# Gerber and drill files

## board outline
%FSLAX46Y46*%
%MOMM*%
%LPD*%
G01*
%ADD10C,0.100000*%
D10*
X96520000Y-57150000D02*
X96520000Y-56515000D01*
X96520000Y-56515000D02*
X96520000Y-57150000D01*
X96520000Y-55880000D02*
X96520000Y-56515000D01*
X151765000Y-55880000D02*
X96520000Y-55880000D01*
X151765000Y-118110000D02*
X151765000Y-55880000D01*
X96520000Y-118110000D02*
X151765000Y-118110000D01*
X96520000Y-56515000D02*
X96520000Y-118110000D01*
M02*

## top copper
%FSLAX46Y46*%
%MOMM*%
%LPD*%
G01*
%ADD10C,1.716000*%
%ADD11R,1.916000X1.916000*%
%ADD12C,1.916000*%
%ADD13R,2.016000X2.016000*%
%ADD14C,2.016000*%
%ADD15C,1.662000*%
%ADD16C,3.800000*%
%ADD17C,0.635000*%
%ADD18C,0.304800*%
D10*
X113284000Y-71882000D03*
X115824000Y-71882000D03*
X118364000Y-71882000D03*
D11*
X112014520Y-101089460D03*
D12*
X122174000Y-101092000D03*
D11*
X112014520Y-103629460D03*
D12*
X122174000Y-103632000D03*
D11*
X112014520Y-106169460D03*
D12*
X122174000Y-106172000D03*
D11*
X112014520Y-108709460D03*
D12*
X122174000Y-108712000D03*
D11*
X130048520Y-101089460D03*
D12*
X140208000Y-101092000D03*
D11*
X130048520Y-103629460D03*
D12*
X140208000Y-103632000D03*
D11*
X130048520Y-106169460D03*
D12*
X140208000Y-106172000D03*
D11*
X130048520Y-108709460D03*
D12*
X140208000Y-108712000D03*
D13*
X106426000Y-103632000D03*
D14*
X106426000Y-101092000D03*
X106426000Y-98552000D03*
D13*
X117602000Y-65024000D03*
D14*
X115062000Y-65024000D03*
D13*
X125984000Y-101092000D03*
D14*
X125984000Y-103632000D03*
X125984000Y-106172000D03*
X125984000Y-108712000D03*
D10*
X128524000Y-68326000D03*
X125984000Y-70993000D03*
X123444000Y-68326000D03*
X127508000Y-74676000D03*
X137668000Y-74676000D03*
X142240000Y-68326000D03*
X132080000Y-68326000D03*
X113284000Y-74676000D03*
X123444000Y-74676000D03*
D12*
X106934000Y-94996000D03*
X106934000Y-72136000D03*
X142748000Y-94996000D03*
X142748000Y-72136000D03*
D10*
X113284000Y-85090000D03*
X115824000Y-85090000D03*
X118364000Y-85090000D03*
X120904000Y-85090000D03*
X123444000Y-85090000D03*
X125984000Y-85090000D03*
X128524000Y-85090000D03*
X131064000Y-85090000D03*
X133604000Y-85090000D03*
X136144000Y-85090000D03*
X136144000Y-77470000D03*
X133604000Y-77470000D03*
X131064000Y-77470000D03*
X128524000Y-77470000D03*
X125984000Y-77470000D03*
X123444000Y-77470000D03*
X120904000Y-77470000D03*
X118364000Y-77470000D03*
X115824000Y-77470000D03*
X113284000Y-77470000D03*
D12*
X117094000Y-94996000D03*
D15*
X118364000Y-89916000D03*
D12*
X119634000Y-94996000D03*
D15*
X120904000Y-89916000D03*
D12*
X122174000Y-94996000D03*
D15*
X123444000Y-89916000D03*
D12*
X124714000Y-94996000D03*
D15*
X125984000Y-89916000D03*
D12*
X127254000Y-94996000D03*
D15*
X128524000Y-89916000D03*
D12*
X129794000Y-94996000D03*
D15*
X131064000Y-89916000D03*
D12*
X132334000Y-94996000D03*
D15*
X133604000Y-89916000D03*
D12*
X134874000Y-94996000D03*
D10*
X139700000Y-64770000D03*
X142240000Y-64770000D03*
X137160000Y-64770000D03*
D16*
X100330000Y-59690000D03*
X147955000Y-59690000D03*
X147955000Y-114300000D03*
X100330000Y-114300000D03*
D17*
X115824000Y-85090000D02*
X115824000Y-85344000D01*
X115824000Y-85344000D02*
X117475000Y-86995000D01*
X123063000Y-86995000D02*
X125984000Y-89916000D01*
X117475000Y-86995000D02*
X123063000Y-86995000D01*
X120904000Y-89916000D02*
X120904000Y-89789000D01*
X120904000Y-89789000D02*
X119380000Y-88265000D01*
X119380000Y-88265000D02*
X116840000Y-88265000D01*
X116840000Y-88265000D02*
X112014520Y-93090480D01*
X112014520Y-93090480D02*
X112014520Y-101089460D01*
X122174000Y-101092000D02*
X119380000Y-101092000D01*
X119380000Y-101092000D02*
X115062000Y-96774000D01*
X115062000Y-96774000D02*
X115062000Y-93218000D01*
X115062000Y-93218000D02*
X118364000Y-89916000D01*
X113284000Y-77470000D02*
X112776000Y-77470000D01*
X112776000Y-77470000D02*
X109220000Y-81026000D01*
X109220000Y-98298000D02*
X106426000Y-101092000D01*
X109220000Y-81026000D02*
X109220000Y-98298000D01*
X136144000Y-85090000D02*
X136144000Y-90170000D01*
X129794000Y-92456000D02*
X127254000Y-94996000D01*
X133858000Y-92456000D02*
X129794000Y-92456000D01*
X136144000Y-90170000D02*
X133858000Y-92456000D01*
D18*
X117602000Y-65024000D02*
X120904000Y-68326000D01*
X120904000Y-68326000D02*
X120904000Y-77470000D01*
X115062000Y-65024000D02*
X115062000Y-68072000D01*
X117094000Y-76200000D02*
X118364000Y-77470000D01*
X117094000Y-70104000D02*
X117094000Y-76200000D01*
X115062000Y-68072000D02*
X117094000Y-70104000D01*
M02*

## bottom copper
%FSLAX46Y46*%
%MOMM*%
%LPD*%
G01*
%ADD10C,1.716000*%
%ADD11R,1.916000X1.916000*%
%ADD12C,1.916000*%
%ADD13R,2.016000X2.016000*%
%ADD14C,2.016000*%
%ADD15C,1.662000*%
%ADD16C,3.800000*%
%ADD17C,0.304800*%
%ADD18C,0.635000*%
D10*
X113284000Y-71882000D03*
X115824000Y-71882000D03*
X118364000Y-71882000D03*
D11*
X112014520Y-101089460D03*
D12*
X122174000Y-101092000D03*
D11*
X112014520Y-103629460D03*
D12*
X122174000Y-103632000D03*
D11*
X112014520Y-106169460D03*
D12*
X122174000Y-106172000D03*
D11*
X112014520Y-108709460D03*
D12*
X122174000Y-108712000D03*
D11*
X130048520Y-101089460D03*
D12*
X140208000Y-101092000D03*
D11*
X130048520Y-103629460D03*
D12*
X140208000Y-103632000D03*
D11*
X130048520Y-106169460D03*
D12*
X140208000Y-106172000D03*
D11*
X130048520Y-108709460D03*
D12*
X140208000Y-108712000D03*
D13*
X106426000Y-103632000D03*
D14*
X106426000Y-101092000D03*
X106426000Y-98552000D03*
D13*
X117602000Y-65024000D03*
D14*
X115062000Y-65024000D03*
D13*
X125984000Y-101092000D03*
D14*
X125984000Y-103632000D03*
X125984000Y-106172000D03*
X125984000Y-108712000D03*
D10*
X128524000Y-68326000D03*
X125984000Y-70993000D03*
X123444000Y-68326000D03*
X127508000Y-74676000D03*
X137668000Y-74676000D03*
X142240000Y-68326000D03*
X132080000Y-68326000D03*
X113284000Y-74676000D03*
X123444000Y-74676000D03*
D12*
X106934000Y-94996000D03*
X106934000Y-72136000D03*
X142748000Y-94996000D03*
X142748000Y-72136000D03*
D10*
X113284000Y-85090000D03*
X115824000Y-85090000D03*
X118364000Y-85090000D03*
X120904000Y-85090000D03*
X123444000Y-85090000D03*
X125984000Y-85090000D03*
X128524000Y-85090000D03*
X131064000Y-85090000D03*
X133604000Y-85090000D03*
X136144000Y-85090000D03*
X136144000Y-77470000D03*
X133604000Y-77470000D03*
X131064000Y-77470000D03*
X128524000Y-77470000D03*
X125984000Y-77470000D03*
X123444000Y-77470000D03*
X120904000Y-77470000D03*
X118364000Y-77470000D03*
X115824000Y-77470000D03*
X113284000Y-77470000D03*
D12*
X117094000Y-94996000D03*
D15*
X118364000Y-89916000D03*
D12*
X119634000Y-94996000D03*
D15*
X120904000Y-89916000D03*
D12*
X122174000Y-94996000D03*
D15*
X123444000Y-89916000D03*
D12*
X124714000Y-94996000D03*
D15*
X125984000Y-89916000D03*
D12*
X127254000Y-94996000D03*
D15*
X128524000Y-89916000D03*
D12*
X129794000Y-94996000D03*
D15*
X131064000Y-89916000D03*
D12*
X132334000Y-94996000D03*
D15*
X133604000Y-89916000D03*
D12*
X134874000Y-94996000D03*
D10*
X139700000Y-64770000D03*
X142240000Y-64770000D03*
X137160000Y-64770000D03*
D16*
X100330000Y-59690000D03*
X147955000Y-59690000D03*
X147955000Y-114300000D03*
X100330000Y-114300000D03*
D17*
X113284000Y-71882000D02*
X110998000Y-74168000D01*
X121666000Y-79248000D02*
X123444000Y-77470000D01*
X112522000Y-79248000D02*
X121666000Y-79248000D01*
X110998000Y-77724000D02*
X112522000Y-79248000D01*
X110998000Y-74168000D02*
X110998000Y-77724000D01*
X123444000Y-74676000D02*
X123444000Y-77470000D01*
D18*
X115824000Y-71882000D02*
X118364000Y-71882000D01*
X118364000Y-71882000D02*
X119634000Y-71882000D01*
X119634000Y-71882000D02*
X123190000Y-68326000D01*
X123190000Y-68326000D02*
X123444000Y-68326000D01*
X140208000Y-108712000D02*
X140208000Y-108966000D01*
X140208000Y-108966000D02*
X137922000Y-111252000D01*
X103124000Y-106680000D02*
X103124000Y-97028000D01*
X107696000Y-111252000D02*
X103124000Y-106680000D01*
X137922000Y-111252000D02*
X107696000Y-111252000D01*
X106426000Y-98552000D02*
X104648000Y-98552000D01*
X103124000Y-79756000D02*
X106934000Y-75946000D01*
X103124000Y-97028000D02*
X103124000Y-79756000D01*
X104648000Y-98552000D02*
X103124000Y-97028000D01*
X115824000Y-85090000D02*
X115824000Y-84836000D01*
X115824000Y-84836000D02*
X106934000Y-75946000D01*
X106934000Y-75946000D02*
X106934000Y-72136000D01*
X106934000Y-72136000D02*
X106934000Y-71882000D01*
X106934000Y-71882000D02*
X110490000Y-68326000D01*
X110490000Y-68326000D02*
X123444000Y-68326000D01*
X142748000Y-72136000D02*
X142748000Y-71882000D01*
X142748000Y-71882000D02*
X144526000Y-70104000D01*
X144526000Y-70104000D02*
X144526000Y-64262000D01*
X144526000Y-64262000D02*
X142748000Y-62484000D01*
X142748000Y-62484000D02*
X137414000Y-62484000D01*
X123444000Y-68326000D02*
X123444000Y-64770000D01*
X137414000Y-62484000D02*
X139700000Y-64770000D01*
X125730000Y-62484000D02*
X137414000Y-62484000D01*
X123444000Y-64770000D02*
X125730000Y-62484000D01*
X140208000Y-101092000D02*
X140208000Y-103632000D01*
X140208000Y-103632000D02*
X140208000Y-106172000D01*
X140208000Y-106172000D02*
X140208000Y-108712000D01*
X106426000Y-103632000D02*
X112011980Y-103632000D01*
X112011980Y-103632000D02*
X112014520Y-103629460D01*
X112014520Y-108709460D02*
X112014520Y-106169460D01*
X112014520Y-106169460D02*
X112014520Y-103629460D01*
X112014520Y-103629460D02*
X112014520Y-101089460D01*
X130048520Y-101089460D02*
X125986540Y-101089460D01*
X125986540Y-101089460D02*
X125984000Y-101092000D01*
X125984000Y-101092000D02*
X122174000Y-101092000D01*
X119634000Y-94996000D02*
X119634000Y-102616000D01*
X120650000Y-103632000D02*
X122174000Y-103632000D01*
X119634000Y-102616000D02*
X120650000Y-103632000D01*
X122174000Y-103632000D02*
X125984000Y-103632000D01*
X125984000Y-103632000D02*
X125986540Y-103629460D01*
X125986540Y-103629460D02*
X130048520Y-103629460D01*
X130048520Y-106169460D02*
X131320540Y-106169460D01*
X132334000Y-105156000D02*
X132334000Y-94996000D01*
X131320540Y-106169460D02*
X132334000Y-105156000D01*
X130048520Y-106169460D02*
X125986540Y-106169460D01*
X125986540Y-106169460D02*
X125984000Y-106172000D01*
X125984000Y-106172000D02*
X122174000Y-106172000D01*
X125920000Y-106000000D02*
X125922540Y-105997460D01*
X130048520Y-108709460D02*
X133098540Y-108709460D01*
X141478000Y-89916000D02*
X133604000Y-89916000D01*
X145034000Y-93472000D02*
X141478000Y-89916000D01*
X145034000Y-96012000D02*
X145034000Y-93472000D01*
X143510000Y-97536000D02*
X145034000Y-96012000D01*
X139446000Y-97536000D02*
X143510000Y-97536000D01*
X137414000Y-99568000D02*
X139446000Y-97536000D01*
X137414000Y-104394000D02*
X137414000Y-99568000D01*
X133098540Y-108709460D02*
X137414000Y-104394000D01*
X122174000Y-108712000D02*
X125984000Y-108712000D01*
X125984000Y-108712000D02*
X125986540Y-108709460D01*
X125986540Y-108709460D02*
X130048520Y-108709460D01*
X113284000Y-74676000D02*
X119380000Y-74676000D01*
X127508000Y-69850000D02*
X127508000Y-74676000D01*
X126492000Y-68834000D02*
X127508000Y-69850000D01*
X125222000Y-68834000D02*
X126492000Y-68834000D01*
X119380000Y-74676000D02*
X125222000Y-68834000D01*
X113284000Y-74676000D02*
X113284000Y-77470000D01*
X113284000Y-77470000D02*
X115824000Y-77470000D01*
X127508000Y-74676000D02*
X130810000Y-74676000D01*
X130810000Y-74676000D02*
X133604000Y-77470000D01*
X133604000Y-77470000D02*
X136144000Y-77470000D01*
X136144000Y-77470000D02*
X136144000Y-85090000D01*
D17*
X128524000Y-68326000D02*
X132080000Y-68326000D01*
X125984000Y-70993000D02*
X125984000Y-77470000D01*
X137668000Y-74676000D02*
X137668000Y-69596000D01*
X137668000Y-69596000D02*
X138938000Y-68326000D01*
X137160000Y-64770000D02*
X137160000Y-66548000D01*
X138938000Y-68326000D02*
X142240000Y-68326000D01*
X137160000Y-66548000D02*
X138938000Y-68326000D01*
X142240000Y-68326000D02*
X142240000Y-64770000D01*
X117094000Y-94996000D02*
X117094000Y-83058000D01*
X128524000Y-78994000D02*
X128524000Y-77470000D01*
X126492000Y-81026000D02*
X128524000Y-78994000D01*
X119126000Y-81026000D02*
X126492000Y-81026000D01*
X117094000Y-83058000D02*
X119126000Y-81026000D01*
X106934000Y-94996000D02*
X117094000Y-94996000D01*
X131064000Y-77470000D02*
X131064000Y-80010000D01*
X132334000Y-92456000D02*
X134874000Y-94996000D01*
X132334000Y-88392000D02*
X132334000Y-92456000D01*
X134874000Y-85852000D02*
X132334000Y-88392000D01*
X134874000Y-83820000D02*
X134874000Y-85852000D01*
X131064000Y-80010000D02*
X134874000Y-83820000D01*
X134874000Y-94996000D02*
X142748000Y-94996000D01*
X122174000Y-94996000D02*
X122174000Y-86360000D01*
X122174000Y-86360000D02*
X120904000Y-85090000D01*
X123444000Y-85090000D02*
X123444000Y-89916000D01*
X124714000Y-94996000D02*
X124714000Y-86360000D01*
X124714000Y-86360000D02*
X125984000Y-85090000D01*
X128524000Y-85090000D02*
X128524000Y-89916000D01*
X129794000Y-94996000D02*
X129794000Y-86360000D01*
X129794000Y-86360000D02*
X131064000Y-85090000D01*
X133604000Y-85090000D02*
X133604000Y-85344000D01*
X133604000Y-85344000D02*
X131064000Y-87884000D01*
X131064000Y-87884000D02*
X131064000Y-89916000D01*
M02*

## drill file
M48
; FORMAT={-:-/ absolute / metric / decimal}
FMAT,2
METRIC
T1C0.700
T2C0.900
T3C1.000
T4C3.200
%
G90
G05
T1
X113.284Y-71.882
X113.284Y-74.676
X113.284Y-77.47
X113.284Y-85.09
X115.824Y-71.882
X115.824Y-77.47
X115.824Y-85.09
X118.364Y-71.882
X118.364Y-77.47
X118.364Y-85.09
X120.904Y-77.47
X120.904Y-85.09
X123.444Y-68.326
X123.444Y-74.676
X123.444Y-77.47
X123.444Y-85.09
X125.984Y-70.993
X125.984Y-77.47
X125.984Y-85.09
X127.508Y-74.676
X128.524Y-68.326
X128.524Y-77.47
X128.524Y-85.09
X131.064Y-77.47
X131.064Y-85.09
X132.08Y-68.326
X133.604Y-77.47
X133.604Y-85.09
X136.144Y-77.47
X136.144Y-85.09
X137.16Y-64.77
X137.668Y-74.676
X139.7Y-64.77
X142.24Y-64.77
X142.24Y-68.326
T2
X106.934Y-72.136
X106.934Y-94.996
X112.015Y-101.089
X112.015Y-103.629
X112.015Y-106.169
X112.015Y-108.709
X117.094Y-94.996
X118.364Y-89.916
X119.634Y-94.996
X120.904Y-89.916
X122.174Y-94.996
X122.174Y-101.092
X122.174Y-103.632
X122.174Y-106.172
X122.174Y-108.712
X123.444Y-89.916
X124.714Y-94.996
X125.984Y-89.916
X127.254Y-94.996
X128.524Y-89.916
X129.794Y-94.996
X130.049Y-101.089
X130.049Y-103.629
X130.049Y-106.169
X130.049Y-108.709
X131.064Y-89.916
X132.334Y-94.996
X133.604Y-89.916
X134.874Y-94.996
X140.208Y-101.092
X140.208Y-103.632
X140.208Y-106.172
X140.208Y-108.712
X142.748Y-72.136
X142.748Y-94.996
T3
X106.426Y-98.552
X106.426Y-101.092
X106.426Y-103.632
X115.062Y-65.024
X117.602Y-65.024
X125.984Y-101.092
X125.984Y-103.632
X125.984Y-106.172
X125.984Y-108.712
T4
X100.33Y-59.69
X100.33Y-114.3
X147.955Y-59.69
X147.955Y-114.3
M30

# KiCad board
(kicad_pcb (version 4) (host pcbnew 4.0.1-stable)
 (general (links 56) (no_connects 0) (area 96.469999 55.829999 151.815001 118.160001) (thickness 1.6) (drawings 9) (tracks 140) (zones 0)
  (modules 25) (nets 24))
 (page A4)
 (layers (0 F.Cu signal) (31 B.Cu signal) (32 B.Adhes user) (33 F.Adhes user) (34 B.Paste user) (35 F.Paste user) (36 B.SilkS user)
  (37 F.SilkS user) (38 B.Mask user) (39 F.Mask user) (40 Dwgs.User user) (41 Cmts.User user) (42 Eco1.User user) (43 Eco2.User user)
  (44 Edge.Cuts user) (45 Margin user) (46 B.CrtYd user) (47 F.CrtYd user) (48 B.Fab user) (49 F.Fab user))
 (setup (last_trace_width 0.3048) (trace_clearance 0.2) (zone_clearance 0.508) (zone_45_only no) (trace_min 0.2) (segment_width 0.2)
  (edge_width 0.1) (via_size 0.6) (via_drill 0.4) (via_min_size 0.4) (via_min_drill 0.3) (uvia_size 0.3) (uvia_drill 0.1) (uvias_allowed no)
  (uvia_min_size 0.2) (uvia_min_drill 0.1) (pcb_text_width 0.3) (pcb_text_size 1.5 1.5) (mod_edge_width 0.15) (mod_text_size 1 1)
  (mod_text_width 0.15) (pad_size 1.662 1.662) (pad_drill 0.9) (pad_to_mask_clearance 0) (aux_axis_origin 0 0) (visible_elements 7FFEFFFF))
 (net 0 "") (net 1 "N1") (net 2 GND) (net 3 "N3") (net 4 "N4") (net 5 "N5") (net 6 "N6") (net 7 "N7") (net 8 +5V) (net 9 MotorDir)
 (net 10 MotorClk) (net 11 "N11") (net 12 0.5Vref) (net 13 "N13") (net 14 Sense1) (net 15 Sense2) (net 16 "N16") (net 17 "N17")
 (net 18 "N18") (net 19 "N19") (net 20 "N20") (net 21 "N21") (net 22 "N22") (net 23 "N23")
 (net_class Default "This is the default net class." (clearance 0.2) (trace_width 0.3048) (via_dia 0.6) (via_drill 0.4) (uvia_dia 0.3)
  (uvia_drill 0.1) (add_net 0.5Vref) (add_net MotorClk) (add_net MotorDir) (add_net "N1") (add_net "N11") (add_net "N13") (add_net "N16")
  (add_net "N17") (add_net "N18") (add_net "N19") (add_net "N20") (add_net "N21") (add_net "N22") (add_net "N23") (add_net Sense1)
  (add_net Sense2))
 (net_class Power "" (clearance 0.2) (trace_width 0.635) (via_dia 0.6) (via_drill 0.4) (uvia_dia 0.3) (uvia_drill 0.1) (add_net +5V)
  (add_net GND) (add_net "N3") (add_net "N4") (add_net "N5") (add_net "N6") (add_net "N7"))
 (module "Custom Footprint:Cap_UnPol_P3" (layer F.Cu) (at 113.284 71.882 90)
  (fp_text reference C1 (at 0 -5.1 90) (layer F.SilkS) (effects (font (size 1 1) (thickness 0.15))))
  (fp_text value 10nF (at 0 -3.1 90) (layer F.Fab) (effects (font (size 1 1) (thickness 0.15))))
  (pad 1 thru_hole circle (at 0 0 90) (size 1.716 1.716) (drill 0.7) (layers *.Cu *.Mask F.SilkS) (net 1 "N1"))
  (pad 2 thru_hole circle (at 0 2.54 90) (size 1.716 1.716) (drill 0.7) (layers *.Cu *.Mask F.SilkS) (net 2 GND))
  (pad 2 thru_hole circle (at 0 5.08 90) (size 1.716 1.716) (drill 0.7) (layers *.Cu *.Mask F.SilkS) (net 2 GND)))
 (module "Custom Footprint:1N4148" (layer F.Cu) (at 112.014 101.092)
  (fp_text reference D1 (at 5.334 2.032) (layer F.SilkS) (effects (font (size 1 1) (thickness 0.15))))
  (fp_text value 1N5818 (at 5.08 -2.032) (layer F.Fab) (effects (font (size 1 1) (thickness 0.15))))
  (pad 1 thru_hole rect (at 0.00052 -0.00254 180) (size 1.916 1.916) (drill 0.9) (layers *.Cu *.Mask F.SilkS) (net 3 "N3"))
  (pad 2 thru_hole circle (at 10.16 0) (size 1.916 1.916) (drill 0.9) (layers *.Cu *.Mask F.SilkS) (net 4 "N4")))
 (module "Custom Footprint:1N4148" (layer F.Cu) (at 112.014 103.632)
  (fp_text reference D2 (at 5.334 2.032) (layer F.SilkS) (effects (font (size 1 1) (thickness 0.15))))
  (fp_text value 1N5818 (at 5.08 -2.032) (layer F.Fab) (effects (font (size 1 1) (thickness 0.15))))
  (pad 1 thru_hole rect (at 0.00052 -0.00254 180) (size 1.916 1.916) (drill 0.9) (layers *.Cu *.Mask F.SilkS) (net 3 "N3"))
  (pad 2 thru_hole circle (at 10.16 0) (size 1.916 1.916) (drill 0.9) (layers *.Cu *.Mask F.SilkS) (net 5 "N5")))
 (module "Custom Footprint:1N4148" (layer F.Cu) (at 112.014 106.172)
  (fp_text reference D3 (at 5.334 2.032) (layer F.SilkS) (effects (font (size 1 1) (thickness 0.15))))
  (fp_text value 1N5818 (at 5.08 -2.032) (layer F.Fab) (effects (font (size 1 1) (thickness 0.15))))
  (pad 1 thru_hole rect (at 0.00052 -0.00254 180) (size 1.916 1.916) (drill 0.9) (layers *.Cu *.Mask F.SilkS) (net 3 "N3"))
  (pad 2 thru_hole circle (at 10.16 0) (size 1.916 1.916) (drill 0.9) (layers *.Cu *.Mask F.SilkS) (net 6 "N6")))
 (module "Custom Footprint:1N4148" (layer F.Cu) (at 112.014 108.712)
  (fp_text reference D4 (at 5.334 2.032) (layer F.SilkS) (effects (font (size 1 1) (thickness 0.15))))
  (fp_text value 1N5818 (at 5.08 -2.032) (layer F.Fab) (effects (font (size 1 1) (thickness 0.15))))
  (pad 1 thru_hole rect (at 0.00052 -0.00254 180) (size 1.916 1.916) (drill 0.9) (layers *.Cu *.Mask F.SilkS) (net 3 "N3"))
  (pad 2 thru_hole circle (at 10.16 0) (size 1.916 1.916) (drill 0.9) (layers *.Cu *.Mask F.SilkS) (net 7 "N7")))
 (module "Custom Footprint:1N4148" (layer F.Cu) (at 130.048 101.092)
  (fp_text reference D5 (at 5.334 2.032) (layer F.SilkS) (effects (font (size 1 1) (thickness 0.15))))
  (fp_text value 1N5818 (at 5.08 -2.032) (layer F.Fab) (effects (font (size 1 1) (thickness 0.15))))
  (pad 1 thru_hole rect (at 0.00052 -0.00254 180) (size 1.916 1.916) (drill 0.9) (layers *.Cu *.Mask F.SilkS) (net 4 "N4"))
  (pad 2 thru_hole circle (at 10.16 0) (size 1.916 1.916) (drill 0.9) (layers *.Cu *.Mask F.SilkS) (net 2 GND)))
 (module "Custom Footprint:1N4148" (layer F.Cu) (at 130.048 103.632)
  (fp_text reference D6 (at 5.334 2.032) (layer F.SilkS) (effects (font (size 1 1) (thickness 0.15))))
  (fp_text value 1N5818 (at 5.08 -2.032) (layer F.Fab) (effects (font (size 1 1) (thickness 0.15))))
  (pad 1 thru_hole rect (at 0.00052 -0.00254 180) (size 1.916 1.916) (drill 0.9) (layers *.Cu *.Mask F.SilkS) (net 5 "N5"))
  (pad 2 thru_hole circle (at 10.16 0) (size 1.916 1.916) (drill 0.9) (layers *.Cu *.Mask F.SilkS) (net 2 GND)))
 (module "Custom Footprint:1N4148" (layer F.Cu) (at 130.048 106.172)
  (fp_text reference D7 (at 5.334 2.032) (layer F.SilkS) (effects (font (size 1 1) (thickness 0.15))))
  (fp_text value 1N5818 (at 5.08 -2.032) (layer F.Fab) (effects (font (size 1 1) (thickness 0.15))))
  (pad 1 thru_hole rect (at 0.00052 -0.00254 180) (size 1.916 1.916) (drill 0.9) (layers *.Cu *.Mask F.SilkS) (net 6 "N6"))
  (pad 2 thru_hole circle (at 10.16 0) (size 1.916 1.916) (drill 0.9) (layers *.Cu *.Mask F.SilkS) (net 2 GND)))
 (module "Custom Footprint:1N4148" (layer F.Cu) (at 130.048 108.712)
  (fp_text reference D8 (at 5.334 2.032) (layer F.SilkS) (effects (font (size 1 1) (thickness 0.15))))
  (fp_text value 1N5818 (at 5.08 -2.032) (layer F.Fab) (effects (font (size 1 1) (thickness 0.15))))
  (pad 1 thru_hole rect (at 0.00052 -0.00254 180) (size 1.916 1.916) (drill 0.9) (layers *.Cu *.Mask F.SilkS) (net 7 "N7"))
  (pad 2 thru_hole circle (at 10.16 0) (size 1.916 1.916) (drill 0.9) (layers *.Cu *.Mask F.SilkS) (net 2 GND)))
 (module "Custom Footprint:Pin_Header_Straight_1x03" (layer F.Cu) (at 106.426 103.632 180)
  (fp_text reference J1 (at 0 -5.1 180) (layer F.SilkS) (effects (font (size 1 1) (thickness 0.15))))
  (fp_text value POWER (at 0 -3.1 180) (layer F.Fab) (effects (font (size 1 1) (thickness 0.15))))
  (pad 1 thru_hole rect (at 0 0 180) (size 2.016 2.016) (drill 1) (layers *.Cu *.Mask F.SilkS) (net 3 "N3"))
  (pad 2 thru_hole circle (at 0 2.54 180) (size 2.016 2.016) (drill 1) (layers *.Cu *.Mask F.SilkS) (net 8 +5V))
  (pad 3 thru_hole circle (at 0 5.08 180) (size 2.016 2.016) (drill 1) (layers *.Cu *.Mask F.SilkS) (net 2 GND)))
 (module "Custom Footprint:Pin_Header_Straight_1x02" (layer F.Cu) (at 117.602 65.024 270)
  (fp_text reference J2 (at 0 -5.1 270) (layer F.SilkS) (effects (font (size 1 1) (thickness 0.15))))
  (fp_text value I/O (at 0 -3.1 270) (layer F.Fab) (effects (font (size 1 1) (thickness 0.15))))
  (pad 1 thru_hole rect (at 0 0 270) (size 2.016 2.016) (drill 1) (layers *.Cu *.Mask F.SilkS) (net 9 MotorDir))
  (pad 2 thru_hole circle (at 0 2.54 270) (size 2.016 2.016) (drill 1) (layers *.Cu *.Mask F.SilkS) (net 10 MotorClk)))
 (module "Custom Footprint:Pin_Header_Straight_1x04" (layer F.Cu) (at 125.984 101.092)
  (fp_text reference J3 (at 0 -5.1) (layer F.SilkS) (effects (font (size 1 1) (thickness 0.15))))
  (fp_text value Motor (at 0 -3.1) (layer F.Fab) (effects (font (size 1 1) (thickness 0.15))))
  (pad 1 thru_hole rect (at 0 0) (size 2.016 2.016) (drill 1) (layers *.Cu *.Mask F.SilkS) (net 4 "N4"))
  (pad 2 thru_hole circle (at 0 2.54) (size 2.016 2.016) (drill 1) (layers *.Cu *.Mask F.SilkS) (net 5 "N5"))
  (pad 3 thru_hole circle (at 0 5.08) (size 2.016 2.016) (drill 1) (layers *.Cu *.Mask F.SilkS) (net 6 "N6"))
  (pad 4 thru_hole circle (at 0 7.62) (size 2.016 2.016) (drill 1) (layers *.Cu *.Mask F.SilkS) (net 7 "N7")))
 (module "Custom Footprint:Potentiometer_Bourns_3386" (layer F.Cu) (at 128.524 68.326)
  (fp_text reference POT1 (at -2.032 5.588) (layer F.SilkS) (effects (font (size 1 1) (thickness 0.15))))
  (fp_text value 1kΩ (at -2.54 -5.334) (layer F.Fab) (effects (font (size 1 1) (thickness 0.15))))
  (pad 1 thru_hole circle (at 0 0) (size 1.716 1.716) (drill 0.7) (layers *.Cu *.Mask F.SilkS) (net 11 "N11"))
  (pad 2 thru_hole circle (at -2.54 2.667) (size 1.716 1.716) (drill 0.7) (layers *.Cu *.Mask F.SilkS) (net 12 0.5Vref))
  (pad 3 thru_hole circle (at -5.08 0) (size 1.716 1.716) (drill 0.7) (layers *.Cu *.Mask F.SilkS) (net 2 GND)))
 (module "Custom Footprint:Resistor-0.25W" (layer F.Cu) (at 127.508 74.676)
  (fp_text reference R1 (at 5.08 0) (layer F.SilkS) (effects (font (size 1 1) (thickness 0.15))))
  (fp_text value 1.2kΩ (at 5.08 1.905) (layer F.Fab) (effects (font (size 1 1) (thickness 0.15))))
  (pad 1 thru_hole circle (at 0 0) (size 1.716 1.716) (drill 0.7) (layers *.Cu *.Mask F.SilkS) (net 8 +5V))
  (pad 2 thru_hole circle (at 10.16 0) (size 1.716 1.716) (drill 0.7) (layers *.Cu *.Mask F.SilkS) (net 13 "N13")))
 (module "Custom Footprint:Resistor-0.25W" (layer F.Cu) (at 142.24 68.326 180)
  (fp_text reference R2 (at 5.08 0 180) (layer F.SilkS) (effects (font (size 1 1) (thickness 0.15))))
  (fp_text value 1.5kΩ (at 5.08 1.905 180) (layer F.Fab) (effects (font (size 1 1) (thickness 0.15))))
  (pad 1 thru_hole circle (at 0 0 180) (size 1.716 1.716) (drill 0.7) (layers *.Cu *.Mask F.SilkS) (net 13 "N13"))
  (pad 2 thru_hole circle (at 10.16 0 180) (size 1.716 1.716) (drill 0.7) (layers *.Cu *.Mask F.SilkS) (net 11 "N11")))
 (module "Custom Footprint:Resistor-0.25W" (layer F.Cu) (at 113.284 74.676)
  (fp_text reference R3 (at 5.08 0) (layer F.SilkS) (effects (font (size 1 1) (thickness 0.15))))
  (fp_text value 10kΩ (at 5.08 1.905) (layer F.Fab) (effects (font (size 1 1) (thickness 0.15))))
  (pad 1 thru_hole circle (at 0 0) (size 1.716 1.716) (drill 0.7) (layers *.Cu *.Mask F.SilkS) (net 8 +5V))
  (pad 2 thru_hole circle (at 10.16 0) (size 1.716 1.716) (drill 0.7) (layers *.Cu *.Mask F.SilkS) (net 1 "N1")))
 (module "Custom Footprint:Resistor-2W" (layer F.Cu) (at 106.934 94.996 90)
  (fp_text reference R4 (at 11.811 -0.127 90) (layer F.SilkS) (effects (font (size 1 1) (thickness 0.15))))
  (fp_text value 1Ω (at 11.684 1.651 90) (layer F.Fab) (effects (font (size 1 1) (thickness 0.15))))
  (pad 1 thru_hole circle (at 0 0 90) (size 1.916 1.916) (drill 0.9) (layers *.Cu *.SilkS *.Mask) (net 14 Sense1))
  (pad 2 thru_hole circle (at 22.86 0 90) (size 1.916 1.916) (drill 0.9) (layers *.Cu *.SilkS *.Mask) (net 2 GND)))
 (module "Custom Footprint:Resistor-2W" (layer F.Cu) (at 142.748 94.996 90)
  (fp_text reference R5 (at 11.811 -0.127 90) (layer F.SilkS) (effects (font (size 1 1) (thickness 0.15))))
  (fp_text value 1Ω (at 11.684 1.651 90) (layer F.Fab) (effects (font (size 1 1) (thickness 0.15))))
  (pad 1 thru_hole circle (at 0 0 90) (size 1.916 1.916) (drill 0.9) (layers *.Cu *.SilkS *.Mask) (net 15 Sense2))
  (pad 2 thru_hole circle (at 22.86 0 90) (size 1.916 1.916) (drill 0.9) (layers *.Cu *.SilkS *.Mask) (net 2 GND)))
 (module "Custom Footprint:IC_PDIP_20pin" (layer F.Cu) (at 113.284 85.09 90)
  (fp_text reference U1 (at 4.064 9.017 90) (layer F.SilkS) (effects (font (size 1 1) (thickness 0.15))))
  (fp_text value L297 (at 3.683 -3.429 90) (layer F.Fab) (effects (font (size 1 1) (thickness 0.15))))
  (pad 1 thru_hole circle (at 0 0 90) (size 1.716 1.716) (drill 0.7) (layers *.Cu *.Mask F.SilkS) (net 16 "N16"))
  (pad 2 thru_hole circle (at 0 2.54 90) (size 1.716 1.716) (drill 0.7) (layers *.Cu *.Mask F.SilkS) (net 2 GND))
  (pad 3 thru_hole circle (at 0 5.08 90) (size 1.716 1.716) (drill 0.7) (layers *.Cu *.Mask F.SilkS) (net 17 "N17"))
  (pad 4 thru_hole circle (at 0 7.62 90) (size 1.716 1.716) (drill 0.7) (layers *.Cu *.Mask F.SilkS) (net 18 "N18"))
  (pad 5 thru_hole circle (at 0 10.16 90) (size 1.716 1.716) (drill 0.7) (layers *.Cu *.Mask F.SilkS) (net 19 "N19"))
  (pad 6 thru_hole circle (at 0 12.7 90) (size 1.716 1.716) (drill 0.7) (layers *.Cu *.Mask F.SilkS) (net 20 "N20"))
  (pad 7 thru_hole circle (at 0 15.24 90) (size 1.716 1.716) (drill 0.7) (layers *.Cu *.Mask F.SilkS) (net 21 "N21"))
  (pad 8 thru_hole circle (at 0 17.78 90) (size 1.716 1.716) (drill 0.7) (layers *.Cu *.Mask F.SilkS) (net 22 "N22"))
  (pad 9 thru_hole circle (at 0 20.32 90) (size 1.716 1.716) (drill 0.7) (layers *.Cu *.Mask F.SilkS) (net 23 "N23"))
  (pad 10 thru_hole circle (at 0 22.86 90) (size 1.716 1.716) (drill 0.7) (layers *.Cu *.Mask F.SilkS) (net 8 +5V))
  (pad 11 thru_hole circle (at 7.62 22.86 90) (size 1.716 1.716) (drill 0.7) (layers *.Cu *.Mask F.SilkS) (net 8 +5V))
  (pad 12 thru_hole circle (at 7.62 20.32 90) (size 1.716 1.716) (drill 0.7) (layers *.Cu *.Mask F.SilkS) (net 8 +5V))
  (pad 13 thru_hole circle (at 7.62 17.78 90) (size 1.716 1.716) (drill 0.7) (layers *.Cu *.Mask F.SilkS) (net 15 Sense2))
  (pad 14 thru_hole circle (at 7.62 15.24 90) (size 1.716 1.716) (drill 0.7) (layers *.Cu *.Mask F.SilkS) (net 14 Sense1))
  (pad 15 thru_hole circle (at 7.62 12.7 90) (size 1.716 1.716) (drill 0.7) (layers *.Cu *.Mask F.SilkS) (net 12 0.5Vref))
  (pad 16 thru_hole circle (at 7.62 10.16 90) (size 1.716 1.716) (drill 0.7) (layers *.Cu *.Mask F.SilkS) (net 1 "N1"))
  (pad 17 thru_hole circle (at 7.62 7.62 90) (size 1.716 1.716) (drill 0.7) (layers *.Cu *.Mask F.SilkS) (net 9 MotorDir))
  (pad 18 thru_hole circle (at 7.62 5.08 90) (size 1.716 1.716) (drill 0.7) (layers *.Cu *.Mask F.SilkS) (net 10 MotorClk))
  (pad 19 thru_hole circle (at 7.62 2.54 90) (size 1.716 1.716) (drill 0.7) (layers *.Cu *.Mask F.SilkS) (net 8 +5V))
  (pad 20 thru_hole circle (at 7.62 0 90) (size 1.716 1.716) (drill 0.7) (layers *.Cu *.Mask F.SilkS) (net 8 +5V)))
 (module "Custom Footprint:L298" (layer F.Cu) (at 117.094 89.916)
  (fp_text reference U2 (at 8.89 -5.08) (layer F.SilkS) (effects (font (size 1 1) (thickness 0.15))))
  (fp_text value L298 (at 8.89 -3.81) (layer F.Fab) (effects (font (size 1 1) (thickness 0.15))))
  (pad 1 thru_hole circle (at 0 5.08) (size 1.916 1.916) (drill 0.9) (layers *.Cu *.Mask F.SilkS) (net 14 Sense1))
  (pad 2 thru_hole circle (at 1.27 0) (size 1.662 1.662) (drill 0.9) (layers *.Cu *.Mask F.SilkS) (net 4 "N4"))
  (pad 3 thru_hole circle (at 2.54 5.08) (size 1.916 1.916) (drill 0.9) (layers *.Cu *.Mask F.SilkS) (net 5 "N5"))
  (pad 4 thru_hole circle (at 3.81 0) (size 1.662 1.662) (drill 0.9) (layers *.Cu *.Mask F.SilkS) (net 3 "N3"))
  (pad 5 thru_hole circle (at 5.08 5.08) (size 1.916 1.916) (drill 0.9) (layers *.Cu *.Mask F.SilkS) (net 18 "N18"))
  (pad 6 thru_hole circle (at 6.35 0) (size 1.662 1.662) (drill 0.9) (layers *.Cu *.Mask F.SilkS) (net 19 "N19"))
  (pad 7 thru_hole circle (at 7.62 5.08) (size 1.916 1.916) (drill 0.9) (layers *.Cu *.Mask F.SilkS) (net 20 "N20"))
  (pad 8 thru_hole circle (at 8.89 0) (size 1.662 1.662) (drill 0.9) (layers *.Cu *.Mask F.SilkS) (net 2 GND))
  (pad 9 thru_hole circle (at 10.16 5.08) (size 1.916 1.916) (drill 0.9) (layers *.Cu *.Mask F.SilkS) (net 8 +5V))
  (pad 10 thru_hole circle (at 11.43 0) (size 1.662 1.662) (drill 0.9) (layers *.Cu *.Mask F.SilkS) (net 21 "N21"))
  (pad 11 thru_hole circle (at 12.7 5.08) (size 1.916 1.916) (drill 0.9) (layers *.Cu *.Mask F.SilkS) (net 22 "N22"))
  (pad 12 thru_hole circle (at 13.97 0) (size 1.662 1.662) (drill 0.9) (layers *.Cu *.Mask F.SilkS) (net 23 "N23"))
  (pad 13 thru_hole circle (at 15.24 5.08) (size 1.916 1.916) (drill 0.9) (layers *.Cu *.Mask F.SilkS) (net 6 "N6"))
  (pad 14 thru_hole circle (at 16.51 0) (size 1.662 1.662) (drill 0.9) (layers *.Cu *.Mask F.SilkS) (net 7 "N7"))
  (pad 15 thru_hole circle (at 17.78 5.08) (size 1.916 1.916) (drill 0.9) (layers *.Cu *.Mask F.SilkS) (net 15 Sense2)))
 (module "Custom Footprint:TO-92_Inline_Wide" (layer F.Cu) (at 137.16 64.77)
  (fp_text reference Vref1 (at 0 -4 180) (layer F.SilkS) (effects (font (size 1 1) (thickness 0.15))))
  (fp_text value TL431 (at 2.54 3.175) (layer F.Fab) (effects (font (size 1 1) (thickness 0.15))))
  (pad 2 thru_hole circle (at 2.54 0 90) (size 1.716 1.716) (drill 0.7) (layers *.Cu *.Mask F.SilkS) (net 2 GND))
  (pad 3 thru_hole circle (at 5.08 0 90) (size 1.716 1.716) (drill 0.7) (layers *.Cu *.Mask F.SilkS) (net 13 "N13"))
  (pad 1 thru_hole circle (at 0 0 90) (size 1.716 1.716) (drill 0.7) (layers *.Cu *.Mask F.SilkS) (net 13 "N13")))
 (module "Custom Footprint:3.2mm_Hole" (layer F.Cu) (at 100.33 59.69)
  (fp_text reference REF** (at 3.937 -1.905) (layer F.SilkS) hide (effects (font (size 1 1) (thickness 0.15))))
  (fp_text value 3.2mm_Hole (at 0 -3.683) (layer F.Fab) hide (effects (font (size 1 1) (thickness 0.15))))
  (pad 1 thru_hole circle (at 0 0) (size 3.8 3.8) (drill 3.2) (layers *.Cu *.Mask F.SilkS)))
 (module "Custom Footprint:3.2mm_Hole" (layer F.Cu) (at 147.955 59.69)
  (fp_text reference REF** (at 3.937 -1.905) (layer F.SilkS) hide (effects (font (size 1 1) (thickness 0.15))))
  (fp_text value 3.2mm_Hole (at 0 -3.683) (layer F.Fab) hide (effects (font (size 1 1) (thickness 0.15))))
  (pad 1 thru_hole circle (at 0 0) (size 3.8 3.8) (drill 3.2) (layers *.Cu *.Mask F.SilkS)))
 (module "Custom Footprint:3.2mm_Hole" (layer F.Cu) (at 147.955 114.3)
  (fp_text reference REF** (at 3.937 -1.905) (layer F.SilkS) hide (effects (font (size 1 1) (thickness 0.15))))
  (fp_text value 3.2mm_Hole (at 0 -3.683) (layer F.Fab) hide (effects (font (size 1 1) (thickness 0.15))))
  (pad 1 thru_hole circle (at 0 0) (size 3.8 3.8) (drill 3.2) (layers *.Cu *.Mask F.SilkS)))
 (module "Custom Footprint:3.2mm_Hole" (layer F.Cu) (at 100.33 114.3)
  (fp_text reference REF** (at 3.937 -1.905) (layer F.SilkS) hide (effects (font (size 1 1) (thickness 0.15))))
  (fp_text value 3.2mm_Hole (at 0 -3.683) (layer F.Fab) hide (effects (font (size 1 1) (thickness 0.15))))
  (pad 1 thru_hole circle (at 0 0) (size 3.8 3.8) (drill 3.2) (layers *.Cu *.Mask F.SilkS)))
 (gr_line (start 96.52 57.15) (end 96.52 56.515) (angle 90) (layer Edge.Cuts) (width 0.1))
 (gr_line (start 96.52 56.515) (end 96.52 57.15) (angle 90) (layer Edge.Cuts) (width 0.1))
 (gr_line (start 96.52 55.88) (end 96.52 56.515) (angle 90) (layer Edge.Cuts) (width 0.1))
 (gr_line (start 151.765 55.88) (end 96.52 55.88) (angle 90) (layer Edge.Cuts) (width 0.1))
 (gr_line (start 151.765 118.11) (end 151.765 55.88) (angle 90) (layer Edge.Cuts) (width 0.1))
 (gr_line (start 96.52 118.11) (end 151.765 118.11) (angle 90) (layer Edge.Cuts) (width 0.1))
 (gr_line (start 96.52 56.515) (end 96.52 118.11) (angle 90) (layer Edge.Cuts) (width 0.1))
 (segment (start 113.284 71.882) (end 110.998 74.168) (width 0.3048) (layer B.Cu) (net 1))
 (segment (start 121.666 79.248) (end 123.444 77.47) (width 0.3048) (layer B.Cu) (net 1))
 (segment (start 112.522 79.248) (end 121.666 79.248) (width 0.3048) (layer B.Cu) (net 1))
 (segment (start 110.998 77.724) (end 112.522 79.248) (width 0.3048) (layer B.Cu) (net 1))
 (segment (start 110.998 74.168) (end 110.998 77.724) (width 0.3048) (layer B.Cu) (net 1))
 (segment (start 123.444 74.676) (end 123.444 77.47) (width 0.3048) (layer B.Cu) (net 1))
 (segment (start 115.824 85.09) (end 115.824 85.344) (width 0.635) (layer F.Cu) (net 2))
 (segment (start 115.824 85.344) (end 117.475 86.995) (width 0.635) (layer F.Cu) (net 2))
 (segment (start 123.063 86.995) (end 125.984 89.916) (width 0.635) (layer F.Cu) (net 2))
 (segment (start 117.475 86.995) (end 123.063 86.995) (width 0.635) (layer F.Cu) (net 2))
 (segment (start 115.824 71.882) (end 118.364 71.882) (width 0.635) (layer B.Cu) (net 2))
 (segment (start 118.364 71.882) (end 119.634 71.882) (width 0.635) (layer B.Cu) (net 2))
 (segment (start 119.634 71.882) (end 123.19 68.326) (width 0.635) (layer B.Cu) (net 2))
 (segment (start 123.19 68.326) (end 123.444 68.326) (width 0.635) (layer B.Cu) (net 2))
 (segment (start 140.208 108.712) (end 140.208 108.966) (width 0.635) (layer B.Cu) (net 2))
 (segment (start 140.208 108.966) (end 137.922 111.252) (width 0.635) (layer B.Cu) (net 2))
 (segment (start 103.124 106.68) (end 103.124 97.028) (width 0.635) (layer B.Cu) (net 2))
 (segment (start 107.696 111.252) (end 103.124 106.68) (width 0.635) (layer B.Cu) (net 2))
 (segment (start 137.922 111.252) (end 107.696 111.252) (width 0.635) (layer B.Cu) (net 2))
 (segment (start 106.426 98.552) (end 104.648 98.552) (width 0.635) (layer B.Cu) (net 2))
 (segment (start 103.124 79.756) (end 106.934 75.946) (width 0.635) (layer B.Cu) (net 2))
 (segment (start 103.124 97.028) (end 103.124 79.756) (width 0.635) (layer B.Cu) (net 2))
 (segment (start 104.648 98.552) (end 103.124 97.028) (width 0.635) (layer B.Cu) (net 2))
 (segment (start 115.824 85.09) (end 115.824 84.836) (width 0.635) (layer B.Cu) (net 2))
 (segment (start 115.824 84.836) (end 106.934 75.946) (width 0.635) (layer B.Cu) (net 2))
 (segment (start 106.934 75.946) (end 106.934 72.136) (width 0.635) (layer B.Cu) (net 2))
 (segment (start 106.934 72.136) (end 106.934 71.882) (width 0.635) (layer B.Cu) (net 2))
 (segment (start 106.934 71.882) (end 110.49 68.326) (width 0.635) (layer B.Cu) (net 2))
 (segment (start 110.49 68.326) (end 123.444 68.326) (width 0.635) (layer B.Cu) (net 2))
 (segment (start 142.748 72.136) (end 142.748 71.882) (width 0.635) (layer B.Cu) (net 2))
 (segment (start 142.748 71.882) (end 144.526 70.104) (width 0.635) (layer B.Cu) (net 2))
 (segment (start 144.526 70.104) (end 144.526 64.262) (width 0.635) (layer B.Cu) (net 2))
 (segment (start 144.526 64.262) (end 142.748 62.484) (width 0.635) (layer B.Cu) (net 2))
 (segment (start 142.748 62.484) (end 137.414 62.484) (width 0.635) (layer B.Cu) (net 2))
 (segment (start 123.444 68.326) (end 123.444 64.77) (width 0.635) (layer B.Cu) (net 2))
 (segment (start 137.414 62.484) (end 139.7 64.77) (width 0.635) (layer B.Cu) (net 2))
 (segment (start 125.73 62.484) (end 137.414 62.484) (width 0.635) (layer B.Cu) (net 2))
 (segment (start 123.444 64.77) (end 125.73 62.484) (width 0.635) (layer B.Cu) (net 2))
 (segment (start 140.208 101.092) (end 140.208 103.632) (width 0.635) (layer B.Cu) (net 2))
 (segment (start 140.208 103.632) (end 140.208 106.172) (width 0.635) (layer B.Cu) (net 2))
 (segment (start 140.208 106.172) (end 140.208 108.712) (width 0.635) (layer B.Cu) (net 2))
 (segment (start 120.904 89.916) (end 120.904 89.789) (width 0.635) (layer F.Cu) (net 3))
 (segment (start 120.904 89.789) (end 119.38 88.265) (width 0.635) (layer F.Cu) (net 3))
 (segment (start 119.38 88.265) (end 116.84 88.265) (width 0.635) (layer F.Cu) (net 3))
 (segment (start 116.84 88.265) (end 112.01452 93.09048) (width 0.635) (layer F.Cu) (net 3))
 (segment (start 112.01452 93.09048) (end 112.01452 101.08946) (width 0.635) (layer F.Cu) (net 3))
 (segment (start 106.426 103.632) (end 112.01198 103.632) (width 0.635) (layer B.Cu) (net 3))
 (segment (start 112.01198 103.632) (end 112.01452 103.62946) (width 0.635) (layer B.Cu) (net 3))
 (segment (start 112.01452 108.70946) (end 112.01452 106.16946) (width 0.635) (layer B.Cu) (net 3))
 (segment (start 112.01452 106.16946) (end 112.01452 103.62946) (width 0.635) (layer B.Cu) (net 3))
 (segment (start 112.01452 103.62946) (end 112.01452 101.08946) (width 0.635) (layer B.Cu) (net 3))
 (segment (start 122.174 101.092) (end 119.38 101.092) (width 0.635) (layer F.Cu) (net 4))
 (segment (start 119.38 101.092) (end 115.062 96.774) (width 0.635) (layer F.Cu) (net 4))
 (segment (start 115.062 96.774) (end 115.062 93.218) (width 0.635) (layer F.Cu) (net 4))
 (segment (start 115.062 93.218) (end 118.364 89.916) (width 0.635) (layer F.Cu) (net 4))
 (segment (start 130.04852 101.08946) (end 125.98654 101.08946) (width 0.635) (layer B.Cu) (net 4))
 (segment (start 125.98654 101.08946) (end 125.984 101.092) (width 0.635) (layer B.Cu) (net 4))
 (segment (start 125.984 101.092) (end 122.174 101.092) (width 0.635) (layer B.Cu) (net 4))
 (segment (start 119.634 94.996) (end 119.634 102.616) (width 0.635) (layer B.Cu) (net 5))
 (segment (start 120.65 103.632) (end 122.174 103.632) (width 0.635) (layer B.Cu) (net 5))
 (segment (start 119.634 102.616) (end 120.65 103.632) (width 0.635) (layer B.Cu) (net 5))
 (segment (start 122.174 103.632) (end 125.984 103.632) (width 0.635) (layer B.Cu) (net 5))
 (segment (start 125.984 103.632) (end 125.98654 103.62946) (width 0.635) (layer B.Cu) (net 5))
 (segment (start 125.98654 103.62946) (end 130.04852 103.62946) (width 0.635) (layer B.Cu) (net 5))
 (segment (start 130.04852 106.16946) (end 131.32054 106.16946) (width 0.635) (layer B.Cu) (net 6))
 (segment (start 132.334 105.156) (end 132.334 94.996) (width 0.635) (layer B.Cu) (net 6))
 (segment (start 131.32054 106.16946) (end 132.334 105.156) (width 0.635) (layer B.Cu) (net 6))
 (segment (start 130.04852 106.16946) (end 125.98654 106.16946) (width 0.635) (layer B.Cu) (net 6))
 (segment (start 125.98654 106.16946) (end 125.984 106.172) (width 0.635) (layer B.Cu) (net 6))
 (segment (start 125.984 106.172) (end 122.174 106.172) (width 0.635) (layer B.Cu) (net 6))
 (segment (start 125.92 106) (end 125.92254 105.99746) (width 0.635) (layer B.Cu) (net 6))
 (segment (start 130.04852 108.70946) (end 133.09854 108.70946) (width 0.635) (layer B.Cu) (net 7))
 (segment (start 141.478 89.916) (end 133.604 89.916) (width 0.635) (layer B.Cu) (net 7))
 (segment (start 145.034 93.472) (end 141.478 89.916) (width 0.635) (layer B.Cu) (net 7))
 (segment (start 145.034 96.012) (end 145.034 93.472) (width 0.635) (layer B.Cu) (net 7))
 (segment (start 143.51 97.536) (end 145.034 96.012) (width 0.635) (layer B.Cu) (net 7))
 (segment (start 139.446 97.536) (end 143.51 97.536) (width 0.635) (layer B.Cu) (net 7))
 (segment (start 137.414 99.568) (end 139.446 97.536) (width 0.635) (layer B.Cu) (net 7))
 (segment (start 137.414 104.394) (end 137.414 99.568) (width 0.635) (layer B.Cu) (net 7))
 (segment (start 133.09854 108.70946) (end 137.414 104.394) (width 0.635) (layer B.Cu) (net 7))
 (segment (start 122.174 108.712) (end 125.984 108.712) (width 0.635) (layer B.Cu) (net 7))
 (segment (start 125.984 108.712) (end 125.98654 108.70946) (width 0.635) (layer B.Cu) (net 7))
 (segment (start 125.98654 108.70946) (end 130.04852 108.70946) (width 0.635) (layer B.Cu) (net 7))
 (segment (start 113.284 77.47) (end 112.776 77.47) (width 0.635) (layer F.Cu) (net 8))
 (segment (start 112.776 77.47) (end 109.22 81.026) (width 0.635) (layer F.Cu) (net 8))
 (segment (start 109.22 98.298) (end 106.426 101.092) (width 0.635) (layer F.Cu) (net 8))
 (segment (start 109.22 81.026) (end 109.22 98.298) (width 0.635) (layer F.Cu) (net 8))
 (segment (start 136.144 85.09) (end 136.144 90.17) (width 0.635) (layer F.Cu) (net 8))
 (segment (start 129.794 92.456) (end 127.254 94.996) (width 0.635) (layer F.Cu) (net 8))
 (segment (start 133.858 92.456) (end 129.794 92.456) (width 0.635) (layer F.Cu) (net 8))
 (segment (start 136.144 90.17) (end 133.858 92.456) (width 0.635) (layer F.Cu) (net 8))
 (segment (start 113.284 74.676) (end 119.38 74.676) (width 0.635) (layer B.Cu) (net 8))
 (segment (start 127.508 69.85) (end 127.508 74.676) (width 0.635) (layer B.Cu) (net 8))
 (segment (start 126.492 68.834) (end 127.508 69.85) (width 0.635) (layer B.Cu) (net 8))
 (segment (start 125.222 68.834) (end 126.492 68.834) (width 0.635) (layer B.Cu) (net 8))
 (segment (start 119.38 74.676) (end 125.222 68.834) (width 0.635) (layer B.Cu) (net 8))
 (segment (start 113.284 74.676) (end 113.284 77.47) (width 0.635) (layer B.Cu) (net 8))
 (segment (start 113.284 77.47) (end 115.824 77.47) (width 0.635) (layer B.Cu) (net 8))
 (segment (start 127.508 74.676) (end 130.81 74.676) (width 0.635) (layer B.Cu) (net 8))
 (segment (start 130.81 74.676) (end 133.604 77.47) (width 0.635) (layer B.Cu) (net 8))
 (segment (start 133.604 77.47) (end 136.144 77.47) (width 0.635) (layer B.Cu) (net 8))
 (segment (start 136.144 77.47) (end 136.144 85.09) (width 0.635) (layer B.Cu) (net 8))
 (segment (start 117.602 65.024) (end 120.904 68.326) (width 0.3048) (layer F.Cu) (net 9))
 (segment (start 120.904 68.326) (end 120.904 77.47) (width 0.3048) (layer F.Cu) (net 9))
 (segment (start 115.062 65.024) (end 115.062 68.072) (width 0.3048) (layer F.Cu) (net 10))
 (segment (start 117.094 76.2) (end 118.364 77.47) (width 0.3048) (layer F.Cu) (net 10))
 (segment (start 117.094 70.104) (end 117.094 76.2) (width 0.3048) (layer F.Cu) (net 10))
 (segment (start 115.062 68.072) (end 117.094 70.104) (width 0.3048) (layer F.Cu) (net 10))
 (segment (start 128.524 68.326) (end 132.08 68.326) (width 0.3048) (layer B.Cu) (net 11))
 (segment (start 125.984 70.993) (end 125.984 77.47) (width 0.3048) (layer B.Cu) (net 12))
 (segment (start 137.668 74.676) (end 137.668 69.596) (width 0.3048) (layer B.Cu) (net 13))
 (segment (start 137.668 69.596) (end 138.938 68.326) (width 0.3048) (layer B.Cu) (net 13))
 (segment (start 137.16 64.77) (end 137.16 66.548) (width 0.3048) (layer B.Cu) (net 13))
 (segment (start 138.938 68.326) (end 142.24 68.326) (width 0.3048) (layer B.Cu) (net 13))
 (segment (start 137.16 66.548) (end 138.938 68.326) (width 0.3048) (layer B.Cu) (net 13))
 (segment (start 142.24 68.326) (end 142.24 64.77) (width 0.3048) (layer B.Cu) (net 13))
 (segment (start 117.094 94.996) (end 117.094 83.058) (width 0.3048) (layer B.Cu) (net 14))
 (segment (start 128.524 78.994) (end 128.524 77.47) (width 0.3048) (layer B.Cu) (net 14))
 (segment (start 126.492 81.026) (end 128.524 78.994) (width 0.3048) (layer B.Cu) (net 14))
 (segment (start 119.126 81.026) (end 126.492 81.026) (width 0.3048) (layer B.Cu) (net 14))
 (segment (start 117.094 83.058) (end 119.126 81.026) (width 0.3048) (layer B.Cu) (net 14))
 (segment (start 106.934 94.996) (end 117.094 94.996) (width 0.3048) (layer B.Cu) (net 14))
 (segment (start 131.064 77.47) (end 131.064 80.01) (width 0.3048) (layer B.Cu) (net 15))
 (segment (start 132.334 92.456) (end 134.874 94.996) (width 0.3048) (layer B.Cu) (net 15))
 (segment (start 132.334 88.392) (end 132.334 92.456) (width 0.3048) (layer B.Cu) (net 15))
 (segment (start 134.874 85.852) (end 132.334 88.392) (width 0.3048) (layer B.Cu) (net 15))
 (segment (start 134.874 83.82) (end 134.874 85.852) (width 0.3048) (layer B.Cu) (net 15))
 (segment (start 131.064 80.01) (end 134.874 83.82) (width 0.3048) (layer B.Cu) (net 15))
 (segment (start 134.874 94.996) (end 142.748 94.996) (width 0.3048) (layer B.Cu) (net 15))
 (segment (start 122.174 94.996) (end 122.174 86.36) (width 0.3048) (layer B.Cu) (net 18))
 (segment (start 122.174 86.36) (end 120.904 85.09) (width 0.3048) (layer B.Cu) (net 18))
 (segment (start 123.444 85.09) (end 123.444 89.916) (width 0.3048) (layer B.Cu) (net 19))
 (segment (start 124.714 94.996) (end 124.714 86.36) (width 0.3048) (layer B.Cu) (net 20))
 (segment (start 124.714 86.36) (end 125.984 85.09) (width 0.3048) (layer B.Cu) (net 20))
 (segment (start 128.524 85.09) (end 128.524 89.916) (width 0.3048) (layer B.Cu) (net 21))
 (segment (start 129.794 94.996) (end 129.794 86.36) (width 0.3048) (layer B.Cu) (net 22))
 (segment (start 129.794 86.36) (end 131.064 85.09) (width 0.3048) (layer B.Cu) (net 22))
 (segment (start 133.604 85.09) (end 133.604 85.344) (width 0.3048) (layer B.Cu) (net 23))
 (segment (start 133.604 85.344) (end 131.064 87.884) (width 0.3048) (layer B.Cu) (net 23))
 (segment (start 131.064 87.884) (end 131.064 89.916) (width 0.3048) (layer B.Cu) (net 23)))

